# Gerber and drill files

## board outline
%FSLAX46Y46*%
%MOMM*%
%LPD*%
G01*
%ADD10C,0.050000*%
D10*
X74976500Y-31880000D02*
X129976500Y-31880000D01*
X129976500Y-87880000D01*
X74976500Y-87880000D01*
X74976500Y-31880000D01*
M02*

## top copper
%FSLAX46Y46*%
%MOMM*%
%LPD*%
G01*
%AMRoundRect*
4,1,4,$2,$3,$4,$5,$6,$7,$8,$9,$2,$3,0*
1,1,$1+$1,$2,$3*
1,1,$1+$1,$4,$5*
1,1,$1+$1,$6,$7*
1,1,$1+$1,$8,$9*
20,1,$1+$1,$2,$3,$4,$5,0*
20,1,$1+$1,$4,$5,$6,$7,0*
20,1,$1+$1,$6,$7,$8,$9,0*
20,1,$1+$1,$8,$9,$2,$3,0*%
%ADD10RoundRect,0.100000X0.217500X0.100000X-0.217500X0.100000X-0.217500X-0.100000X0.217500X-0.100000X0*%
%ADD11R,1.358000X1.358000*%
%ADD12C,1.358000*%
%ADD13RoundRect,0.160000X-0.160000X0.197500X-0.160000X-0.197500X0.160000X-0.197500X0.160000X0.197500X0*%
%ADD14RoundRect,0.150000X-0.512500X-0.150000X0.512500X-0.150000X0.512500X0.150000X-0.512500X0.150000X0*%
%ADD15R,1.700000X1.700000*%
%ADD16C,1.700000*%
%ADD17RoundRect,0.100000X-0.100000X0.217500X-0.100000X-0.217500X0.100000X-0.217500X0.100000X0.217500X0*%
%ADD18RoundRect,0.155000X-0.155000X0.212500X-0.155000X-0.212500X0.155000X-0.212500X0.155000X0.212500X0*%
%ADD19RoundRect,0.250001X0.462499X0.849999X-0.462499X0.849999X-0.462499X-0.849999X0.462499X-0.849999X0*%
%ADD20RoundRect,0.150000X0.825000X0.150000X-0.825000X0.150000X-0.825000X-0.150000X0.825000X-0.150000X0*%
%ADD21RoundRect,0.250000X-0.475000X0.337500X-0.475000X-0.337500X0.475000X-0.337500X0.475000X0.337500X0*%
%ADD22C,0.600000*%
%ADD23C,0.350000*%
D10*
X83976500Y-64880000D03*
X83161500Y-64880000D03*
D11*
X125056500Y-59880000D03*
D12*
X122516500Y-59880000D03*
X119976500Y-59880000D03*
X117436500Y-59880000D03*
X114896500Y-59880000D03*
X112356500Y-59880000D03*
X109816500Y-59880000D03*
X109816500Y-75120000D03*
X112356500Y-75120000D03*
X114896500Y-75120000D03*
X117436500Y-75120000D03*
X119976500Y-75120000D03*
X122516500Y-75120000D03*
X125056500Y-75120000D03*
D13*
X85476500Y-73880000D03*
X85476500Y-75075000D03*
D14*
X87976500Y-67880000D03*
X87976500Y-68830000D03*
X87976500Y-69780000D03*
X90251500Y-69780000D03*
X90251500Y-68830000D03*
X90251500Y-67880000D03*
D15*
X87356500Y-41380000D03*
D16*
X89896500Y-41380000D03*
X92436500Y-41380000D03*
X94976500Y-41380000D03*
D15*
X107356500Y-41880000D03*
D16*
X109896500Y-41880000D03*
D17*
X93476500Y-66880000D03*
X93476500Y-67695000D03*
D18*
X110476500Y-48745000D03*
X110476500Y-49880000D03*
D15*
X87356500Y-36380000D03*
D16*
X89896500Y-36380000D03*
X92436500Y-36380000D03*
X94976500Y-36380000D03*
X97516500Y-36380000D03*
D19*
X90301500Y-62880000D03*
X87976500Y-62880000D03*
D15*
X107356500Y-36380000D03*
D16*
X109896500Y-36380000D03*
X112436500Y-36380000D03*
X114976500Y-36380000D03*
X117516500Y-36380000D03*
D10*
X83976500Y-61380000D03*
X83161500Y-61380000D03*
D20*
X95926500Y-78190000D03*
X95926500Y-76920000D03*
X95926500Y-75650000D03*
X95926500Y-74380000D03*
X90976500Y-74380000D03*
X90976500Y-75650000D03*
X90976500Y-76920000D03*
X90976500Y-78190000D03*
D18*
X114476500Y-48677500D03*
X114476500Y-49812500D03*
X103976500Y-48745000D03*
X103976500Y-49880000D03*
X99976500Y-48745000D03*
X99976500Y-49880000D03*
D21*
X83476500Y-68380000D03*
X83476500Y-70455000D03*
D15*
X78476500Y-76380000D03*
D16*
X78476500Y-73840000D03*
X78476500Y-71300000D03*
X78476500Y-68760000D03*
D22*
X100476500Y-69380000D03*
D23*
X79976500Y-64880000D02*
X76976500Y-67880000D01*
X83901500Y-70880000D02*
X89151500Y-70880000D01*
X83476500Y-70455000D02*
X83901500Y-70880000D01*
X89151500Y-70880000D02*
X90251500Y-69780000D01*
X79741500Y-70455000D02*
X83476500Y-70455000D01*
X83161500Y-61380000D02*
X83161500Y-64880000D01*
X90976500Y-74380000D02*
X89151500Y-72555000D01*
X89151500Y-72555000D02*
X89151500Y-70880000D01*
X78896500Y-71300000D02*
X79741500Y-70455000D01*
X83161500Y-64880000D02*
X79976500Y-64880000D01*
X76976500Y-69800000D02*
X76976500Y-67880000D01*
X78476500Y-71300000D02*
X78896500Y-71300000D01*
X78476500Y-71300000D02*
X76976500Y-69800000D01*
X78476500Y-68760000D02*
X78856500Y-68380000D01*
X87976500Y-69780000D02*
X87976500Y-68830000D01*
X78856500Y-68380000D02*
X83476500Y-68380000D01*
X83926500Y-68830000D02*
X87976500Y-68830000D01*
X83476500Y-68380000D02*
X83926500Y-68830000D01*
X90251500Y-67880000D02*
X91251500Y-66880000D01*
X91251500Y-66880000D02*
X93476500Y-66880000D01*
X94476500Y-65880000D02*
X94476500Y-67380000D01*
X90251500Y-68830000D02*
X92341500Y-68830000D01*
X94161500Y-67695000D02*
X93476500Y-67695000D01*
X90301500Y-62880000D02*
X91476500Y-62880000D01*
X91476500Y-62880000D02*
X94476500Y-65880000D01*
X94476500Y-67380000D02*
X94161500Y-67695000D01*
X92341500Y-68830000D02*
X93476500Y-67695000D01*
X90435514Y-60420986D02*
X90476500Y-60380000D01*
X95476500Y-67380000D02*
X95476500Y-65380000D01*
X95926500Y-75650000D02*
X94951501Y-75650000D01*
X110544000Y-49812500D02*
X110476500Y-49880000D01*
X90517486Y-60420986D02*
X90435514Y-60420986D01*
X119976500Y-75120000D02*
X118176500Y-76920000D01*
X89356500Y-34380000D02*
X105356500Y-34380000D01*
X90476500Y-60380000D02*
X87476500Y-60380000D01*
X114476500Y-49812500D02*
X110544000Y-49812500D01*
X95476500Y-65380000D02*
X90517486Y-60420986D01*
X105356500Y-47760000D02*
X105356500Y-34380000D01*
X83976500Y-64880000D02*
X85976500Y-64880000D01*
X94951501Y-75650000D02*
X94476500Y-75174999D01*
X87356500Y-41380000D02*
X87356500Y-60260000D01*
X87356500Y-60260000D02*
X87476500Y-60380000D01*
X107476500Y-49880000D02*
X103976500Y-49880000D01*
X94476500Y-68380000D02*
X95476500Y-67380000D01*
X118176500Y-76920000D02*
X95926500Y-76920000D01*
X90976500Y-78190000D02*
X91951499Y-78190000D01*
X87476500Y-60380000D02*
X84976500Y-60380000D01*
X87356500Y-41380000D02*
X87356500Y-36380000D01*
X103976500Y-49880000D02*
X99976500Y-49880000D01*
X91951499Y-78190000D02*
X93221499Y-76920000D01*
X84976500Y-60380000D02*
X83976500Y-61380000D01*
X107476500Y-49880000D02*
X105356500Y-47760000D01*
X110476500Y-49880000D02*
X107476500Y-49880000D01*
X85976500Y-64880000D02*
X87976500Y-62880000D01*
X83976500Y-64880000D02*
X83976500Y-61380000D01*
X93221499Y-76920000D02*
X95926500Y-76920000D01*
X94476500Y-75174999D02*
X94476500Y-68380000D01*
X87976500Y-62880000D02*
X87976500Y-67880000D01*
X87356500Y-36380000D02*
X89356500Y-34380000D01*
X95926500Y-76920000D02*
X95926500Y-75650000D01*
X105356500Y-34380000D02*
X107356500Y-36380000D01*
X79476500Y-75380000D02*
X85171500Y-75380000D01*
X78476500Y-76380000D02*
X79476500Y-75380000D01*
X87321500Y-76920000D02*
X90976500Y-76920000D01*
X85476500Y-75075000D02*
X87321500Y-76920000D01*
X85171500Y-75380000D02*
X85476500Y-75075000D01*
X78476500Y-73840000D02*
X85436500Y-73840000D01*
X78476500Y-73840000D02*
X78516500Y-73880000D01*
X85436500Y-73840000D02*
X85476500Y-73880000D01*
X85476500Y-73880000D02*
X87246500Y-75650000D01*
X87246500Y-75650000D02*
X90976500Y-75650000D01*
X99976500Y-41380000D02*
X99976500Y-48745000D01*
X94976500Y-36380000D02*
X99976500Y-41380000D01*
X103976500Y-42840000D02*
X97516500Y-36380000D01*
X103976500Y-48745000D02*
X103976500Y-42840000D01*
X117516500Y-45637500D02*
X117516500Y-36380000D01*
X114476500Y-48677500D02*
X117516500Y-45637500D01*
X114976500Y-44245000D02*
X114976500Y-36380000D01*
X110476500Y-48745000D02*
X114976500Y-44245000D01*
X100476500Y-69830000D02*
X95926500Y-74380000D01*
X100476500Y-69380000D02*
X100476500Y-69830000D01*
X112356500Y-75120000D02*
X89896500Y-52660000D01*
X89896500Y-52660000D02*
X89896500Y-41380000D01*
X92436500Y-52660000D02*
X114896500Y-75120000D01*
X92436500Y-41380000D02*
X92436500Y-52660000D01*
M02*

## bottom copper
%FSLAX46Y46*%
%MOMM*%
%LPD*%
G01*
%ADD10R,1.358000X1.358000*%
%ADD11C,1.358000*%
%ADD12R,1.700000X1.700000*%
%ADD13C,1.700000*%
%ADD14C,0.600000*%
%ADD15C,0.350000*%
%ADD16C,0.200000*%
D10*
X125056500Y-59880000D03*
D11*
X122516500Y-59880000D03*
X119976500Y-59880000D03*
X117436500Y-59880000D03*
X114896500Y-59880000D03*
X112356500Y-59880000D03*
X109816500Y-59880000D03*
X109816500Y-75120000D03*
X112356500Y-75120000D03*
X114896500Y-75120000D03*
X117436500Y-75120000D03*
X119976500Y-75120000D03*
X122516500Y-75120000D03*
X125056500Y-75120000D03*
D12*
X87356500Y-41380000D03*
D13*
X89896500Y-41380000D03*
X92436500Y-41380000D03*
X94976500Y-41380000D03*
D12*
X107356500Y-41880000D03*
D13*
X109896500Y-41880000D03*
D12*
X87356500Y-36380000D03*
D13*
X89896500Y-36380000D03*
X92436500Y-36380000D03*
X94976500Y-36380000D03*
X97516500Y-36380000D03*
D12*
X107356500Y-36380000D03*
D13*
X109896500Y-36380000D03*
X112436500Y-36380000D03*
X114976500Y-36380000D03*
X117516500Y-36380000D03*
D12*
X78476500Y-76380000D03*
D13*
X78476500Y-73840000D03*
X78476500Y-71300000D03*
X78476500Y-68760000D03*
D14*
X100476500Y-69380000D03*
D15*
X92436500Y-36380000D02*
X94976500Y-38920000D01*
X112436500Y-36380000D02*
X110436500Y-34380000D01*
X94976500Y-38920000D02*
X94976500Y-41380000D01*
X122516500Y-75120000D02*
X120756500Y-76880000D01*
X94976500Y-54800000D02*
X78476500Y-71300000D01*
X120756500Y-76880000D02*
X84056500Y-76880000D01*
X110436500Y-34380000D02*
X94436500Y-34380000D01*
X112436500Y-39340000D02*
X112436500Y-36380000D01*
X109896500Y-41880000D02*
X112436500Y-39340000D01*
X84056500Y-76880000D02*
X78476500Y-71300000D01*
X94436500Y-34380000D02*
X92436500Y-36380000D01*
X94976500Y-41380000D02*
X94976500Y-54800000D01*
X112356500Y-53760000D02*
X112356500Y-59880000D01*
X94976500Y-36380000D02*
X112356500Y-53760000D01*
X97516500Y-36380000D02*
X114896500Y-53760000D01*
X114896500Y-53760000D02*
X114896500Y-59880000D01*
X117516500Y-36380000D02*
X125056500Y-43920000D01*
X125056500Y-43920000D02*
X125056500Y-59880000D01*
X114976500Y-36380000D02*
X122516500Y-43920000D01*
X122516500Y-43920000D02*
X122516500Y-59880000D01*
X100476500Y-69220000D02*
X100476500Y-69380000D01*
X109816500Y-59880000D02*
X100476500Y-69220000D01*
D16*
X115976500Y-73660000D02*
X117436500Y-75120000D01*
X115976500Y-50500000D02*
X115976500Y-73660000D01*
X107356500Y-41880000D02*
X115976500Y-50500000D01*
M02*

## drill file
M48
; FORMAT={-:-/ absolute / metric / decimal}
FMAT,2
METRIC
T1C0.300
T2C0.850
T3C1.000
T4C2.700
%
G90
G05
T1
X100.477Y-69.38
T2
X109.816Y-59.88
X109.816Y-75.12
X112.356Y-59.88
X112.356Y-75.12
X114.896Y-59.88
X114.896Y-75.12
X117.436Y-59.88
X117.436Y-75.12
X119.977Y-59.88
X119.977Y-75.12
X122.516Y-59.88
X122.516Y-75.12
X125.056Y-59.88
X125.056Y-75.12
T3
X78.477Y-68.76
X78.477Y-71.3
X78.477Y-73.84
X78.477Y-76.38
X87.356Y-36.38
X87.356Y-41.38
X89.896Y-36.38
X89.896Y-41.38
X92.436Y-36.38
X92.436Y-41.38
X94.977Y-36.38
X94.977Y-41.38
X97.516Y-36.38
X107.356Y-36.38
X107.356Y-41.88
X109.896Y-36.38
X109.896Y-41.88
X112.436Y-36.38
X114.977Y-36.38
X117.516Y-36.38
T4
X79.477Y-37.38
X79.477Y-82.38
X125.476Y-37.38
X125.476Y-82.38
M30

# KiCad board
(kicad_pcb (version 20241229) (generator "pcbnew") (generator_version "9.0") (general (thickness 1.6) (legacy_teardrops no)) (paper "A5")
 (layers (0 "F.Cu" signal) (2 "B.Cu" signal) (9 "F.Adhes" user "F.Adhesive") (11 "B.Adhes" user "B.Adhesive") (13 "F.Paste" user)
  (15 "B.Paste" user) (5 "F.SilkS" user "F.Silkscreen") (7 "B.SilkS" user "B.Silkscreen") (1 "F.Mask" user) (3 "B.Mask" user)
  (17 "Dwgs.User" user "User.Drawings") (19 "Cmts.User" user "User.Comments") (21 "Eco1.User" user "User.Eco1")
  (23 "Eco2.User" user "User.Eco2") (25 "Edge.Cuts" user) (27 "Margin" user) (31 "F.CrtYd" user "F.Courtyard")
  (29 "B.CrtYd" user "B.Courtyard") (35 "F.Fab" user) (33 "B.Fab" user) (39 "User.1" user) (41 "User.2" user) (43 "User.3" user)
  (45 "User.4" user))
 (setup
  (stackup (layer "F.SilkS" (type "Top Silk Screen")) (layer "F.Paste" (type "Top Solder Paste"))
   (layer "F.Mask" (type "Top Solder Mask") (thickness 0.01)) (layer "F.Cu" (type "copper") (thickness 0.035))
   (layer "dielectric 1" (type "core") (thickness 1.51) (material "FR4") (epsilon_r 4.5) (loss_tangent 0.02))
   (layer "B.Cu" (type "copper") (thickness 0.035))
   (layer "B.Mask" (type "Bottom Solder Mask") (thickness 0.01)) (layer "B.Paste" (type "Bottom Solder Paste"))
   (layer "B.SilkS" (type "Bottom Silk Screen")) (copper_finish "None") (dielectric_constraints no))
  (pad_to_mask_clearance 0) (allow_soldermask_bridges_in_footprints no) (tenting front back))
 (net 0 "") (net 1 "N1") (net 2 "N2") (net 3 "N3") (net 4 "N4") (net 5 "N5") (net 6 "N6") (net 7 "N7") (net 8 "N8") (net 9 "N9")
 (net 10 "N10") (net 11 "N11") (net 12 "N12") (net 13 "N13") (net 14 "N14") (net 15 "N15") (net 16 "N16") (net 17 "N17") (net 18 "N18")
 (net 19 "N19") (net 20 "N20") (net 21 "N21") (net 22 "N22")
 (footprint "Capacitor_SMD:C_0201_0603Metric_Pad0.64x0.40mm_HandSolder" (layer "F.Cu") (at 83.569 64.88 180)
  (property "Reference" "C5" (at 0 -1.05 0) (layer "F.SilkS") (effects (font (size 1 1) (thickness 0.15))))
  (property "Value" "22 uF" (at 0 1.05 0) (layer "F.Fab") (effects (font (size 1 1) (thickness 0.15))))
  (pad "" smd roundrect (at -0.4325 0 180) (size 0.458 0.36) (layers "F.Paste") (roundrect_rratio 0.25))
  (pad "" smd roundrect (at 0.4325 0 180) (size 0.458 0.36) (layers "F.Paste") (roundrect_rratio 0.25))
  (pad "1" smd roundrect (at -0.4075 0 180) (size 0.635 0.4) (layers "F.Cu" "F.Mask") (roundrect_rratio 0.25) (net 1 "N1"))
  (pad "2" smd roundrect (at 0.4075 0 180) (size 0.635 0.4) (layers "F.Cu" "F.Mask") (roundrect_rratio 0.25) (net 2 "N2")))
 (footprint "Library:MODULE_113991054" (layer "F.Cu") (at 117.5 67.5 -90)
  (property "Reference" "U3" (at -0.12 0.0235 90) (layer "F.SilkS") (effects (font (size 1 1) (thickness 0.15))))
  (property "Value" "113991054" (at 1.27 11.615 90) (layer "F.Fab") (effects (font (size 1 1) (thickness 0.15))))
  (pad "1" thru_hole rect (at -7.62 -7.5565 270) (size 1.358 1.358) (drill 0.85) (layers "*.Cu" "*.Mask") (remove_unused_layers no)
   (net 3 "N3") (solder_mask_margin 0.102))
  (pad "2" thru_hole circle (at -7.62 -5.0165 270) (size 1.358 1.358) (drill 0.85) (layers "*.Cu" "*.Mask") (remove_unused_layers no)
   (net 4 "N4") (solder_mask_margin 0.102))
  (pad "3" thru_hole circle (at -7.62 -2.4765 270) (size 1.358 1.358) (drill 0.85) (layers "*.Cu" "*.Mask") (remove_unused_layers no)
   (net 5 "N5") (solder_mask_margin 0.102))
  (pad "4" thru_hole circle (at -7.62 0.0635 270) (size 1.358 1.358) (drill 0.85) (layers "*.Cu" "*.Mask") (remove_unused_layers no)
   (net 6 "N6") (solder_mask_margin 0.102))
  (pad "5" thru_hole circle (at -7.62 2.6035 270) (size 1.358 1.358) (drill 0.85) (layers "*.Cu" "*.Mask") (remove_unused_layers no)
   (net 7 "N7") (solder_mask_margin 0.102))
  (pad "6" thru_hole circle (at -7.62 5.1435 270) (size 1.358 1.358) (drill 0.85) (layers "*.Cu" "*.Mask") (remove_unused_layers no)
   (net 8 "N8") (solder_mask_margin 0.102))
  (pad "7" thru_hole circle (at -7.62 7.6835 270) (size 1.358 1.358) (drill 0.85) (layers "*.Cu" "*.Mask") (remove_unused_layers no)
   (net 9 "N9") (solder_mask_margin 0.102))
  (pad "8" thru_hole circle (at 7.62 7.6835 270) (size 1.358 1.358) (drill 0.85) (layers "*.Cu" "*.Mask") (remove_unused_layers no)
   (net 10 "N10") (solder_mask_margin 0.102))
  (pad "9" thru_hole circle (at 7.62 5.1435 270) (size 1.358 1.358) (drill 0.85) (layers "*.Cu" "*.Mask") (remove_unused_layers no)
   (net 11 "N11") (solder_mask_margin 0.102))
  (pad "10" thru_hole circle (at 7.62 2.6035 270) (size 1.358 1.358) (drill 0.85) (layers "*.Cu" "*.Mask") (remove_unused_layers no)
   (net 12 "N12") (solder_mask_margin 0.102))
  (pad "11" thru_hole circle (at 7.62 0.0635 270) (size 1.358 1.358) (drill 0.85) (layers "*.Cu" "*.Mask") (remove_unused_layers no)
   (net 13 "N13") (solder_mask_margin 0.102))
  (pad "12" thru_hole circle (at 7.62 -2.4765 270) (size 1.358 1.358) (drill 0.85) (layers "*.Cu" "*.Mask") (remove_unused_layers no)
   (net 1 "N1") (solder_mask_margin 0.102))
  (pad "13" thru_hole circle (at 7.62 -5.0165 270) (size 1.358 1.358) (drill 0.85) (layers "*.Cu" "*.Mask") (remove_unused_layers no)
   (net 2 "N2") (solder_mask_margin 0.102))
  (pad "14" thru_hole circle (at 7.62 -7.5565 270) (size 1.358 1.358) (drill 0.85) (layers "*.Cu" "*.Mask") (remove_unused_layers no)
   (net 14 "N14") (solder_mask_margin 0.102)))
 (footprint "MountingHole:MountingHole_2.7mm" (layer "F.Cu") (at 125.4765 82.38)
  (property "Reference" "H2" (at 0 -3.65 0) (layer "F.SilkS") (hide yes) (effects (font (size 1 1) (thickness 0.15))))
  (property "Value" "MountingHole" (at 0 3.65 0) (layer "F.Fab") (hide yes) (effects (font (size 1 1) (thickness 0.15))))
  (pad "" np_thru_hole circle (at 0 0) (size 2.7 2.7) (drill 2.7) (layers "*.Cu" "*.Mask")))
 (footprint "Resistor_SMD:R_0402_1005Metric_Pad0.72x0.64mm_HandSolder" (layer "F.Cu") (at 85.4765 74.4775 -90)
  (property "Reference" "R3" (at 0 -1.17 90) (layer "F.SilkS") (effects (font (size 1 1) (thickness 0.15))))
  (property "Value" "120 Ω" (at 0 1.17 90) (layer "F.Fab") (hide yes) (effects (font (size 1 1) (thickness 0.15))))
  (pad "1" smd roundrect (at -0.5975 0 270) (size 0.715 0.64) (layers "F.Cu" "F.Mask" "F.Paste") (roundrect_rratio 0.25) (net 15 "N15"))
  (pad "2" smd roundrect (at 0.5975 0 270) (size 0.715 0.64) (layers "F.Cu" "F.Mask" "F.Paste") (roundrect_rratio 0.25) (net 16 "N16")))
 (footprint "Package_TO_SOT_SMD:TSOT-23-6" (layer "F.Cu") (at 89.114 68.83)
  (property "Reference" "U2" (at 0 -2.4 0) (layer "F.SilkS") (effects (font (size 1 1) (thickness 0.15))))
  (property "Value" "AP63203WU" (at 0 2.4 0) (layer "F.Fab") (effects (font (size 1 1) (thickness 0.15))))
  (pad "1" smd roundrect (at -1.1375 -0.95) (size 1.325 0.6) (layers "F.Cu" "F.Mask" "F.Paste") (roundrect_rratio 0.25) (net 1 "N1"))
  (pad "2" smd roundrect (at -1.1375 0) (size 1.325 0.6) (layers "F.Cu" "F.Mask" "F.Paste") (roundrect_rratio 0.25) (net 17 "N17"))
  (pad "3" smd roundrect (at -1.1375 0.95) (size 1.325 0.6) (layers "F.Cu" "F.Mask" "F.Paste") (roundrect_rratio 0.25) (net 17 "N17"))
  (pad "4" smd roundrect (at 1.1375 0.95) (size 1.325 0.6) (layers "F.Cu" "F.Mask" "F.Paste") (roundrect_rratio 0.25) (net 2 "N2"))
  (pad "5" smd roundrect (at 1.1375 0) (size 1.325 0.6) (layers "F.Cu" "F.Mask" "F.Paste") (roundrect_rratio 0.25) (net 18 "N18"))
  (pad "6" smd roundrect (at 1.1375 -0.95) (size 1.325 0.6) (layers "F.Cu" "F.Mask" "F.Paste") (roundrect_rratio 0.25) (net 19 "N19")))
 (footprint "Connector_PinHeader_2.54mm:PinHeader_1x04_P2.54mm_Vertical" (layer "F.Cu") (at 87.3565 41.38 90)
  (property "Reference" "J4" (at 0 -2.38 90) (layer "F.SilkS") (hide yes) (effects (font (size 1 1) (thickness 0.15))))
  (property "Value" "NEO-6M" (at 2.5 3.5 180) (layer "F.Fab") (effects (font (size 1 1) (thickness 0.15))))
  (pad "1" thru_hole rect (at 0 0 90) (size 1.7 1.7) (drill 1) (layers "*.Cu" "*.Mask") (remove_unused_layers no) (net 1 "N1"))
  (pad "2" thru_hole circle (at 0 2.54 90) (size 1.7 1.7) (drill 1) (layers "*.Cu" "*.Mask") (remove_unused_layers no) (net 11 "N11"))
  (pad "3" thru_hole circle (at 0 5.08 90) (size 1.7 1.7) (drill 1) (layers "*.Cu" "*.Mask") (remove_unused_layers no) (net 12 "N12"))
  (pad "4" thru_hole circle (at 0 7.62 90) (size 1.7 1.7) (drill 1) (layers "*.Cu" "*.Mask") (remove_unused_layers no) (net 2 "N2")))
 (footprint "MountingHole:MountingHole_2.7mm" (layer "F.Cu") (at 79.4765 37.38)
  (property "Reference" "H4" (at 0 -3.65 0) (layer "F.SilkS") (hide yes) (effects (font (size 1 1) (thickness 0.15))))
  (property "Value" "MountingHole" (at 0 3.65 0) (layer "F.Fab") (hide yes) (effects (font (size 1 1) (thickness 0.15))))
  (pad "" np_thru_hole circle (at 0 0) (size 2.7 2.7) (drill 2.7) (layers "*.Cu" "*.Mask")))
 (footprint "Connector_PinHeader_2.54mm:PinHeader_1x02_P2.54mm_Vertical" (layer "F.Cu") (at 107.3565 41.88 90)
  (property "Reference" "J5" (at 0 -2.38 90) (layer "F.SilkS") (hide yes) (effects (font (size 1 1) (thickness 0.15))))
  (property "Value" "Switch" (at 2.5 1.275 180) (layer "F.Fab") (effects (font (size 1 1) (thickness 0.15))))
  (pad "1" thru_hole rect (at 0 0 90) (size 1.7 1.7) (drill 1) (layers "*.Cu" "*.Mask") (remove_unused_layers no) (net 13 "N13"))
  (pad "2" thru_hole circle (at 0 2.54 90) (size 1.7 1.7) (drill 1) (layers "*.Cu" "*.Mask") (remove_unused_layers no) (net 2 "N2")))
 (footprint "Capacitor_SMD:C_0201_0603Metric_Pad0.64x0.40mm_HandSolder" (layer "F.Cu") (at 93.4765 67.2875 -90)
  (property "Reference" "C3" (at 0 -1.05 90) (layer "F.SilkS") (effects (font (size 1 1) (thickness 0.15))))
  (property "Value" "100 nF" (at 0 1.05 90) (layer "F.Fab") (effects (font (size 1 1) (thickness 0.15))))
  (pad "" smd roundrect (at -0.4325 0 270) (size 0.458 0.36) (layers "F.Paste") (roundrect_rratio 0.25))
  (pad "" smd roundrect (at 0.4325 0 270) (size 0.458 0.36) (layers "F.Paste") (roundrect_rratio 0.25))
  (pad "1" smd roundrect (at -0.4075 0 270) (size 0.635 0.4) (layers "F.Cu" "F.Mask") (roundrect_rratio 0.25) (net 19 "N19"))
  (pad "2" smd roundrect (at 0.4075 0 270) (size 0.635 0.4) (layers "F.Cu" "F.Mask") (roundrect_rratio 0.25) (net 18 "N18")))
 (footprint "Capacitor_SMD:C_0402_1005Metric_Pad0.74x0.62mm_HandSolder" (layer "F.Cu") (at 110.4765 49.3125 -90)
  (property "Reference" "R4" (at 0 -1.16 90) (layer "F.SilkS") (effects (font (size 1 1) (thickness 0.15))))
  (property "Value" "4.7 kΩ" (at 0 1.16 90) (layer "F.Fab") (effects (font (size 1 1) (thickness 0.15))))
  (pad "1" smd roundrect (at -0.5675 0 270) (size 0.735 0.62) (layers "F.Cu" "F.Mask" "F.Paste") (roundrect_rratio 0.25) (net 4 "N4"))
  (pad "2" smd roundrect (at 0.5675 0 270) (size 0.735 0.62) (layers "F.Cu" "F.Mask" "F.Paste") (roundrect_rratio 0.25) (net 1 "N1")))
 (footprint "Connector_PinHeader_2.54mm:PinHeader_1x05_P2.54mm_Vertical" (layer "F.Cu") (at 87.3565 36.38 90)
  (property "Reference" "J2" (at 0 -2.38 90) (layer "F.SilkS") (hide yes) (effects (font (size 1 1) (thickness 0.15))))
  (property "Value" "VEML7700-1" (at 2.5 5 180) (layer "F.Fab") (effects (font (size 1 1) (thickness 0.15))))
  (pad "1" thru_hole rect (at 0 0 90) (size 1.7 1.7) (drill 1) (layers "*.Cu" "*.Mask") (remove_unused_layers no) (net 1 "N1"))
  (pad "2" thru_hole circle (at 0 2.54 90) (size 1.7 1.7) (drill 1) (layers "*.Cu" "*.Mask") (remove_unused_layers no) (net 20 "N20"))
  (pad "3" thru_hole circle (at 0 5.08 90) (size 1.7 1.7) (drill 1) (layers "*.Cu" "*.Mask") (remove_unused_layers no) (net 2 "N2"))
  (pad "4" thru_hole circle (at 0 7.62 90) (size 1.7 1.7) (drill 1) (layers "*.Cu" "*.Mask") (remove_unused_layers no) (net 8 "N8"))
  (pad "5" thru_hole circle (at 0 10.16 90) (size 1.7 1.7) (drill 1) (layers "*.Cu" "*.Mask") (remove_unused_layers no) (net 7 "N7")))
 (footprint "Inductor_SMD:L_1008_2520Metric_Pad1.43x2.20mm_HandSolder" (layer "F.Cu") (at 89.139 62.88 180)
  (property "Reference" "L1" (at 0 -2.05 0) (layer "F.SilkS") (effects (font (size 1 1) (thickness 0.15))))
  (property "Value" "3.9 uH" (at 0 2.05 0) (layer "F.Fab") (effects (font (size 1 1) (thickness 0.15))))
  (pad "1" smd roundrect (at -1.1625 0 180) (size 1.425 2.2) (layers "F.Cu" "F.Mask" "F.Paste") (roundrect_rratio 0.175439) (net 18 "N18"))
  (pad "2" smd roundrect (at 1.1625 0 180) (size 1.425 2.2) (layers "F.Cu" "F.Mask" "F.Paste") (roundrect_rratio 0.175439) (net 1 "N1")))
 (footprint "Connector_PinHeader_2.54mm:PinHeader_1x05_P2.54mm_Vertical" (layer "F.Cu") (at 107.3565 36.38 90)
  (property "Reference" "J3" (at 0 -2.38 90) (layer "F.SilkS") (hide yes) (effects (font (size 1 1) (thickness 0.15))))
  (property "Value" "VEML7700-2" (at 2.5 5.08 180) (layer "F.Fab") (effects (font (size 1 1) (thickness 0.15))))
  (pad "1" thru_hole rect (at 0 0 90) (size 1.7 1.7) (drill 1) (layers "*.Cu" "*.Mask") (remove_unused_layers no) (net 1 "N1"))
  (pad "2" thru_hole circle (at 0 2.54 90) (size 1.7 1.7) (drill 1) (layers "*.Cu" "*.Mask") (remove_unused_layers no) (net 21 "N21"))
  (pad "3" thru_hole circle (at 0 5.08 90) (size 1.7 1.7) (drill 1) (layers "*.Cu" "*.Mask") (remove_unused_layers no) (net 2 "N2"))
  (pad "4" thru_hole circle (at 0 7.62 90) (size 1.7 1.7) (drill 1) (layers "*.Cu" "*.Mask") (remove_unused_layers no) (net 4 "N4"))
  (pad "5" thru_hole circle (at 0 10.16 90) (size 1.7 1.7) (drill 1) (layers "*.Cu" "*.Mask") (remove_unused_layers no) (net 3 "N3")))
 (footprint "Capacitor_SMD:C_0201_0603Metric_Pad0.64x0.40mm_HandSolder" (layer "F.Cu") (at 83.569 61.38 180)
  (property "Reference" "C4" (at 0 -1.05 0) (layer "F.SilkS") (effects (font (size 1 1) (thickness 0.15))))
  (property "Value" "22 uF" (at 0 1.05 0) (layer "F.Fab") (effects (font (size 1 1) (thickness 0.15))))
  (pad "" smd roundrect (at -0.4325 0 180) (size 0.458 0.36) (layers "F.Paste") (roundrect_rratio 0.25))
  (pad "" smd roundrect (at 0.4325 0 180) (size 0.458 0.36) (layers "F.Paste") (roundrect_rratio 0.25))
  (pad "1" smd roundrect (at -0.4075 0 180) (size 0.635 0.4) (layers "F.Cu" "F.Mask") (roundrect_rratio 0.25) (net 1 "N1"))
  (pad "2" smd roundrect (at 0.4075 0 180) (size 0.635 0.4) (layers "F.Cu" "F.Mask") (roundrect_rratio 0.25) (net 2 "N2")))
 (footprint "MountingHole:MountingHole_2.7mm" (layer "F.Cu") (at 125.4765 37.38)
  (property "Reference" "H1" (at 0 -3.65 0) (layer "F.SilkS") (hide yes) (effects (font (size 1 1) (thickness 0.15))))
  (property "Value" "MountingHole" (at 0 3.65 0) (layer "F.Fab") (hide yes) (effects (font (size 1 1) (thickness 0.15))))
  (pad "" np_thru_hole circle (at 0 0) (size 2.7 2.7) (drill 2.7) (layers "*.Cu" "*.Mask")))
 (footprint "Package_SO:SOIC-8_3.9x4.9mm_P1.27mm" (layer "F.Cu") (at 93.4515 76.285 180)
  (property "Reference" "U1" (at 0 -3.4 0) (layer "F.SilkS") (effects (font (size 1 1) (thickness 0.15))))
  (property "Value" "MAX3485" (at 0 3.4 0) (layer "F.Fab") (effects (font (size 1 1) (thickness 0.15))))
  (pad "1" smd roundrect (at -2.475 -1.905 180) (size 1.95 0.6) (layers "F.Cu" "F.Mask" "F.Paste") (roundrect_rratio 0.25) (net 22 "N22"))
  (pad "2" smd roundrect (at -2.475 -0.635 180) (size 1.95 0.6) (layers "F.Cu" "F.Mask" "F.Paste") (roundrect_rratio 0.25) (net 1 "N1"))
  (pad "3" smd roundrect (at -2.475 0.635 180) (size 1.95 0.6) (layers "F.Cu" "F.Mask" "F.Paste") (roundrect_rratio 0.25) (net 1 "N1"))
  (pad "4" smd roundrect (at -2.475 1.905 180) (size 1.95 0.6) (layers "F.Cu" "F.Mask" "F.Paste") (roundrect_rratio 0.25) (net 9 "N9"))
  (pad "5" smd roundrect (at 2.475 1.905 180) (size 1.95 0.6) (layers "F.Cu" "F.Mask" "F.Paste") (roundrect_rratio 0.25) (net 2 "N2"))
  (pad "6" smd roundrect (at 2.475 0.635 180) (size 1.95 0.6) (layers "F.Cu" "F.Mask" "F.Paste") (roundrect_rratio 0.25) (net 15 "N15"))
  (pad "7" smd roundrect (at 2.475 -0.635 180) (size 1.95 0.6) (layers "F.Cu" "F.Mask" "F.Paste") (roundrect_rratio 0.25) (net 16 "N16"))
  (pad "8" smd roundrect (at 2.475 -1.905 180) (size 1.95 0.6) (layers "F.Cu" "F.Mask" "F.Paste") (roundrect_rratio 0.25) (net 1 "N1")))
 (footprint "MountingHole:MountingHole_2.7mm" (layer "F.Cu") (at 79.4765 82.38)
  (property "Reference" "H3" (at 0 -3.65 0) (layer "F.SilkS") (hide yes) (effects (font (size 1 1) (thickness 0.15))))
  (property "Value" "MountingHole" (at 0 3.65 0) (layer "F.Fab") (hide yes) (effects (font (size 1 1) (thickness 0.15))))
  (pad "" np_thru_hole circle (at 0 0) (size 2.7 2.7) (drill 2.7) (layers "*.Cu" "*.Mask")))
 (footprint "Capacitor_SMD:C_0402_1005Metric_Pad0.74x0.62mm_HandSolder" (layer "F.Cu") (at 114.4765 49.245 -90)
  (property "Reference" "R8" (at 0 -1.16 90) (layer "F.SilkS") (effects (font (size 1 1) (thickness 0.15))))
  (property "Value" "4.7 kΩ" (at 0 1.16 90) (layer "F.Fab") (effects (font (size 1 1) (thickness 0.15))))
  (pad "1" smd roundrect (at -0.5675 0 270) (size 0.735 0.62) (layers "F.Cu" "F.Mask" "F.Paste") (roundrect_rratio 0.25) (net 3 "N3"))
  (pad "2" smd roundrect (at 0.5675 0 270) (size 0.735 0.62) (layers "F.Cu" "F.Mask" "F.Paste") (roundrect_rratio 0.25) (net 1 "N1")))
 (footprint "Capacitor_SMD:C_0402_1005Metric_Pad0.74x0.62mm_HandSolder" (layer "F.Cu") (at 103.9765 49.3125 -90)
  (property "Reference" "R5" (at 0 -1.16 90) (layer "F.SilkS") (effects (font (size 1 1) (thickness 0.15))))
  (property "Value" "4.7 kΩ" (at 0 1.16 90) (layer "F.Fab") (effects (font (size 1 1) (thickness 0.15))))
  (pad "1" smd roundrect (at -0.5675 0 270) (size 0.735 0.62) (layers "F.Cu" "F.Mask" "F.Paste") (roundrect_rratio 0.25) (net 7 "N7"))
  (pad "2" smd roundrect (at 0.5675 0 270) (size 0.735 0.62) (layers "F.Cu" "F.Mask" "F.Paste") (roundrect_rratio 0.25) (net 1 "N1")))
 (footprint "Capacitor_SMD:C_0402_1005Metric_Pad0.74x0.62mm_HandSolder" (layer "F.Cu") (at 99.9765 49.3125 -90)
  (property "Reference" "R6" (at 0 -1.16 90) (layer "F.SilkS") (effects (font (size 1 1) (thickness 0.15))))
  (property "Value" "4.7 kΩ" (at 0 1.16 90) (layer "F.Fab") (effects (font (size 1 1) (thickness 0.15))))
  (pad "1" smd roundrect (at -0.5675 0 270) (size 0.735 0.62) (layers "F.Cu" "F.Mask" "F.Paste") (roundrect_rratio 0.25) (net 8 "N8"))
  (pad "2" smd roundrect (at 0.5675 0 270) (size 0.735 0.62) (layers "F.Cu" "F.Mask" "F.Paste") (roundrect_rratio 0.25) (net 1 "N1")))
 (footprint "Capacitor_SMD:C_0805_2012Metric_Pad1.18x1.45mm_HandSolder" (layer "F.Cu") (at 83.4765 69.4175 -90)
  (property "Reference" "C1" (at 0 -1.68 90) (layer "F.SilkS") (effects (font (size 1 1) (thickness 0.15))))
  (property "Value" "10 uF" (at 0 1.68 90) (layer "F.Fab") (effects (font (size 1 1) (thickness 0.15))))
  (pad "1" smd roundrect (at -1.0375 0 270) (size 1.175 1.45) (layers "F.Cu" "F.Mask" "F.Paste") (roundrect_rratio 0.212766) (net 17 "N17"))
  (pad "2" smd roundrect (at 1.0375 0 270) (size 1.175 1.45) (layers "F.Cu" "F.Mask" "F.Paste") (roundrect_rratio 0.212766) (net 2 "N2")))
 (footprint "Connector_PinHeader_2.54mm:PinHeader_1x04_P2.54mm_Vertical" (layer "F.Cu") (at 78.4765 76.38 180)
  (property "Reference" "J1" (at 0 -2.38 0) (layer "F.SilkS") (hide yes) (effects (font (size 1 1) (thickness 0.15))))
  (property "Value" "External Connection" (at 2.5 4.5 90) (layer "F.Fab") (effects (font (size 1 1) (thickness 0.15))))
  (pad "1" thru_hole rect (at 0 0 180) (size 1.7 1.7) (drill 1) (layers "*.Cu" "*.Mask") (remove_unused_layers no) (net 16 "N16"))
  (pad "2" thru_hole circle (at 0 2.54 180) (size 1.7 1.7) (drill 1) (layers "*.Cu" "*.Mask") (remove_unused_layers no) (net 15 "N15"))
  (pad "3" thru_hole circle (at 0 5.08 180) (size 1.7 1.7) (drill 1) (layers "*.Cu" "*.Mask") (remove_unused_layers no) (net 2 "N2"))
  (pad "4" thru_hole circle (at 0 7.62 180) (size 1.7 1.7) (drill 1) (layers "*.Cu" "*.Mask") (remove_unused_layers no) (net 17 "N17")))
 (gr_rect (start 74.9765 31.88) (end 129.9765 87.88) (stroke (width 0.05) (type solid)) (fill no) (layer "Edge.Cuts"))
 (segment (start 79.9765 64.88) (end 76.9765 67.88) (width 0.35) (layer "F.Cu") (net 2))
 (segment (start 83.9015 70.88) (end 89.1515 70.88) (width 0.35) (layer "F.Cu") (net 2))
 (segment (start 83.4765 70.455) (end 83.9015 70.88) (width 0.35) (layer "F.Cu") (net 2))
 (segment (start 89.1515 70.88) (end 90.2515 69.78) (width 0.35) (layer "F.Cu") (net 2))
 (segment (start 79.7415 70.455) (end 83.4765 70.455) (width 0.35) (layer "F.Cu") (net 2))
 (segment (start 83.1615 61.38) (end 83.1615 64.88) (width 0.35) (layer "F.Cu") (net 2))
 (segment (start 90.9765 74.38) (end 89.1515 72.555) (width 0.35) (layer "F.Cu") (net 2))
 (segment (start 89.1515 72.555) (end 89.1515 70.88) (width 0.35) (layer "F.Cu") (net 2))
 (segment (start 78.8965 71.3) (end 79.7415 70.455) (width 0.35) (layer "F.Cu") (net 2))
 (segment (start 83.1615 64.88) (end 79.9765 64.88) (width 0.35) (layer "F.Cu") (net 2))
 (segment (start 76.9765 69.8) (end 76.9765 67.88) (width 0.35) (layer "F.Cu") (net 2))
 (segment (start 78.4765 71.3) (end 78.8965 71.3) (width 0.35) (layer "F.Cu") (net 2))
 (segment (start 78.4765 71.3) (end 76.9765 69.8) (width 0.35) (layer "F.Cu") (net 2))
 (segment (start 92.4365 36.38) (end 94.9765 38.92) (width 0.35) (layer "B.Cu") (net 2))
 (segment (start 112.4365 36.38) (end 110.4365 34.38) (width 0.35) (layer "B.Cu") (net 2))
 (segment (start 94.9765 38.92) (end 94.9765 41.38) (width 0.35) (layer "B.Cu") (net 2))
 (segment (start 122.5165 75.12) (end 120.7565 76.88) (width 0.35) (layer "B.Cu") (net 2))
 (segment (start 94.9765 54.8) (end 78.4765 71.3) (width 0.35) (layer "B.Cu") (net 2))
 (segment (start 120.7565 76.88) (end 84.0565 76.88) (width 0.35) (layer "B.Cu") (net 2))
 (segment (start 110.4365 34.38) (end 94.4365 34.38) (width 0.35) (layer "B.Cu") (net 2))
 (segment (start 112.4365 39.34) (end 112.4365 36.38) (width 0.35) (layer "B.Cu") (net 2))
 (segment (start 109.8965 41.88) (end 112.4365 39.34) (width 0.35) (layer "B.Cu") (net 2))
 (segment (start 84.0565 76.88) (end 78.4765 71.3) (width 0.35) (layer "B.Cu") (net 2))
 (segment (start 94.4365 34.38) (end 92.4365 36.38) (width 0.35) (layer "B.Cu") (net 2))
 (segment (start 94.9765 41.38) (end 94.9765 54.8) (width 0.35) (layer "B.Cu") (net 2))
 (segment (start 78.4765 68.76) (end 78.8565 68.38) (width 0.35) (layer "F.Cu") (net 17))
 (segment (start 87.9765 69.78) (end 87.9765 68.83) (width 0.35) (layer "F.Cu") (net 17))
 (segment (start 78.8565 68.38) (end 83.4765 68.38) (width 0.35) (layer "F.Cu") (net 17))
 (segment (start 83.9265 68.83) (end 87.9765 68.83) (width 0.35) (layer "F.Cu") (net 17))
 (segment (start 83.4765 68.38) (end 83.9265 68.83) (width 0.35) (layer "F.Cu") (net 17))
 (segment (start 90.2515 67.88) (end 91.2515 66.88) (width 0.35) (layer "F.Cu") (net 19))
 (segment (start 91.2515 66.88) (end 93.4765 66.88) (width 0.35) (layer "F.Cu") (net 19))
 (segment (start 94.4765 65.88) (end 94.4765 67.38) (width 0.35) (layer "F.Cu") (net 18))
 (segment (start 90.2515 68.83) (end 92.3415 68.83) (width 0.35) (layer "F.Cu") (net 18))
 (segment (start 94.1615 67.695) (end 93.4765 67.695) (width 0.35) (layer "F.Cu") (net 18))
 (segment (start 90.3015 62.88) (end 91.4765 62.88) (width 0.35) (layer "F.Cu") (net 18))
 (segment (start 91.4765 62.88) (end 94.4765 65.88) (width 0.35) (layer "F.Cu") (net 18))
 (segment (start 94.4765 67.38) (end 94.1615 67.695) (width 0.35) (layer "F.Cu") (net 18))
 (segment (start 92.3415 68.83) (end 93.4765 67.695) (width 0.35) (layer "F.Cu") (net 18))
 (segment (start 90.435514 60.420986) (end 90.4765 60.38) (width 0.35) (layer "F.Cu") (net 1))
 (segment (start 95.4765 67.38) (end 95.4765 65.38) (width 0.35) (layer "F.Cu") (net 1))
 (segment (start 95.9265 75.65) (end 94.951501 75.65) (width 0.35) (layer "F.Cu") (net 1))
 (segment (start 110.544 49.8125) (end 110.4765 49.88) (width 0.35) (layer "F.Cu") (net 1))
 (segment (start 90.517486 60.420986) (end 90.435514 60.420986) (width 0.35) (layer "F.Cu") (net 1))
 (segment (start 119.9765 75.12) (end 118.1765 76.92) (width 0.35) (layer "F.Cu") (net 1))
 (segment (start 89.3565 34.38) (end 105.3565 34.38) (width 0.35) (layer "F.Cu") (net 1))
 (segment (start 90.4765 60.38) (end 87.4765 60.38) (width 0.35) (layer "F.Cu") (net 1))
 (segment (start 114.4765 49.8125) (end 110.544 49.8125) (width 0.35) (layer "F.Cu") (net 1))
 (segment (start 95.4765 65.38) (end 90.517486 60.420986) (width 0.35) (layer "F.Cu") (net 1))
 (segment (start 105.3565 47.76) (end 105.3565 34.38) (width 0.35) (layer "F.Cu") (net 1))
 (segment (start 83.9765 64.88) (end 85.9765 64.88) (width 0.35) (layer "F.Cu") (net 1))
 (segment (start 94.951501 75.65) (end 94.4765 75.174999) (width 0.35) (layer "F.Cu") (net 1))
 (segment (start 87.3565 41.38) (end 87.3565 60.26) (width 0.35) (layer "F.Cu") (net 1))
 (segment (start 87.3565 60.26) (end 87.4765 60.38) (width 0.35) (layer "F.Cu") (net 1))
 (segment (start 107.4765 49.88) (end 103.9765 49.88) (width 0.35) (layer "F.Cu") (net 1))
 (segment (start 94.4765 68.38) (end 95.4765 67.38) (width 0.35) (layer "F.Cu") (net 1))
 (segment (start 118.1765 76.92) (end 95.9265 76.92) (width 0.35) (layer "F.Cu") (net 1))
 (segment (start 90.9765 78.19) (end 91.951499 78.19) (width 0.35) (layer "F.Cu") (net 1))
 (segment (start 87.4765 60.38) (end 84.9765 60.38) (width 0.35) (layer "F.Cu") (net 1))
 (segment (start 87.3565 41.38) (end 87.3565 36.38) (width 0.35) (layer "F.Cu") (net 1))
 (segment (start 103.9765 49.88) (end 99.9765 49.88) (width 0.35) (layer "F.Cu") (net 1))
 (segment (start 91.951499 78.19) (end 93.221499 76.92) (width 0.35) (layer "F.Cu") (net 1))
 (segment (start 84.9765 60.38) (end 83.9765 61.38) (width 0.35) (layer "F.Cu") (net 1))
 (segment (start 107.4765 49.88) (end 105.3565 47.76) (width 0.35) (layer "F.Cu") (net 1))
 (segment (start 110.4765 49.88) (end 107.4765 49.88) (width 0.35) (layer "F.Cu") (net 1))
 (segment (start 85.9765 64.88) (end 87.9765 62.88) (width 0.35) (layer "F.Cu") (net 1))
 (segment (start 83.9765 64.88) (end 83.9765 61.38) (width 0.35) (layer "F.Cu") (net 1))
 (segment (start 93.221499 76.92) (end 95.9265 76.92) (width 0.35) (layer "F.Cu") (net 1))
 (segment (start 94.4765 75.174999) (end 94.4765 68.38) (width 0.35) (layer "F.Cu") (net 1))
 (segment (start 87.9765 62.88) (end 87.9765 67.88) (width 0.35) (layer "F.Cu") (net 1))
 (segment (start 87.3565 36.38) (end 89.3565 34.38) (width 0.35) (layer "F.Cu") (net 1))
 (segment (start 95.9265 76.92) (end 95.9265 75.65) (width 0.35) (layer "F.Cu") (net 1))
 (segment (start 105.3565 34.38) (end 107.3565 36.38) (width 0.35) (layer "F.Cu") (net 1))
 (segment (start 79.4765 75.38) (end 85.1715 75.38) (width 0.35) (layer "F.Cu") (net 16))
 (segment (start 78.4765 76.38) (end 79.4765 75.38) (width 0.35) (layer "F.Cu") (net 16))
 (segment (start 87.3215 76.92) (end 90.9765 76.92) (width 0.35) (layer "F.Cu") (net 16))
 (segment (start 85.4765 75.075) (end 87.3215 76.92) (width 0.35) (layer "F.Cu") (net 16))
 (segment (start 85.1715 75.38) (end 85.4765 75.075) (width 0.35) (layer "F.Cu") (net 16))
 (segment (start 78.4765 73.84) (end 85.4365 73.84) (width 0.35) (layer "F.Cu") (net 15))
 (segment (start 78.4765 73.84) (end 78.5165 73.88) (width 0.35) (layer "F.Cu") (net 15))
 (segment (start 85.4365 73.84) (end 85.4765 73.88) (width 0.35) (layer "F.Cu") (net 15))
 (segment (start 85.4765 73.88) (end 87.2465 75.65) (width 0.35) (layer "F.Cu") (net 15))
 (segment (start 87.2465 75.65) (end 90.9765 75.65) (width 0.35) (layer "F.Cu") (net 15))
 (segment (start 99.9765 41.38) (end 99.9765 48.745) (width 0.35) (layer "F.Cu") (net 8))
 (segment (start 94.9765 36.38) (end 99.9765 41.38) (width 0.35) (layer "F.Cu") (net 8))
 (segment (start 112.3565 53.76) (end 112.3565 59.88) (width 0.35) (layer "B.Cu") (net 8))
 (segment (start 94.9765 36.38) (end 112.3565 53.76) (width 0.35) (layer "B.Cu") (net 8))
 (segment (start 103.9765 42.84) (end 97.5165 36.38) (width 0.35) (layer "F.Cu") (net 7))
 (segment (start 103.9765 48.745) (end 103.9765 42.84) (width 0.35) (layer "F.Cu") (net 7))
 (segment (start 97.5165 36.38) (end 114.8965 53.76) (width 0.35) (layer "B.Cu") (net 7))
 (segment (start 114.8965 53.76) (end 114.8965 59.88) (width 0.35) (layer "B.Cu") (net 7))
 (segment (start 117.5165 45.6375) (end 117.5165 36.38) (width 0.35) (layer "F.Cu") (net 3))
 (segment (start 114.4765 48.6775) (end 117.5165 45.6375) (width 0.35) (layer "F.Cu") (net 3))
 (segment (start 117.5165 36.38) (end 125.0565 43.92) (width 0.35) (layer "B.Cu") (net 3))
 (segment (start 125.0565 43.92) (end 125.0565 59.88) (width 0.35) (layer "B.Cu") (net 3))
 (segment (start 114.9765 44.245) (end 114.9765 36.38) (width 0.35) (layer "F.Cu") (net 4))
 (segment (start 110.4765 48.745) (end 114.9765 44.245) (width 0.35) (layer "F.Cu") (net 4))
 (segment (start 114.9765 36.38) (end 122.5165 43.92) (width 0.35) (layer "B.Cu") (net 4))
 (segment (start 122.5165 43.92) (end 122.5165 59.88) (width 0.35) (layer "B.Cu") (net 4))
 (segment (start 100.4765 69.83) (end 95.9265 74.38) (width 0.35) (layer "F.Cu") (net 9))
 (segment (start 100.4765 69.38) (end 100.4765 69.83) (width 0.35) (layer "F.Cu") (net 9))
 (via (at 100.4765 69.38) (size 0.6) (drill 0.3) (layers "F.Cu" "B.Cu") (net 9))
 (segment (start 100.4765 69.22) (end 100.4765 69.38) (width 0.35) (layer "B.Cu") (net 9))
 (segment (start 109.8165 59.88) (end 100.4765 69.22) (width 0.35) (layer "B.Cu") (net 9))
 (segment (start 112.3565 75.12) (end 89.8965 52.66) (width 0.35) (layer "F.Cu") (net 11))
 (segment (start 89.8965 52.66) (end 89.8965 41.38) (width 0.35) (layer "F.Cu") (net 11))
 (segment (start 115.9765 73.66) (end 117.4365 75.12) (width 0.2) (layer "B.Cu") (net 13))
 (segment (start 115.9765 50.5) (end 115.9765 73.66) (width 0.2) (layer "B.Cu") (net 13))
 (segment (start 107.3565 41.88) (end 115.9765 50.5) (width 0.2) (layer "B.Cu") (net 13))
 (segment (start 92.4365 52.66) (end 114.8965 75.12) (width 0.35) (layer "F.Cu") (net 12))
 (segment (start 92.4365 41.38) (end 92.4365 52.66) (width 0.35) (layer "F.Cu") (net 12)))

